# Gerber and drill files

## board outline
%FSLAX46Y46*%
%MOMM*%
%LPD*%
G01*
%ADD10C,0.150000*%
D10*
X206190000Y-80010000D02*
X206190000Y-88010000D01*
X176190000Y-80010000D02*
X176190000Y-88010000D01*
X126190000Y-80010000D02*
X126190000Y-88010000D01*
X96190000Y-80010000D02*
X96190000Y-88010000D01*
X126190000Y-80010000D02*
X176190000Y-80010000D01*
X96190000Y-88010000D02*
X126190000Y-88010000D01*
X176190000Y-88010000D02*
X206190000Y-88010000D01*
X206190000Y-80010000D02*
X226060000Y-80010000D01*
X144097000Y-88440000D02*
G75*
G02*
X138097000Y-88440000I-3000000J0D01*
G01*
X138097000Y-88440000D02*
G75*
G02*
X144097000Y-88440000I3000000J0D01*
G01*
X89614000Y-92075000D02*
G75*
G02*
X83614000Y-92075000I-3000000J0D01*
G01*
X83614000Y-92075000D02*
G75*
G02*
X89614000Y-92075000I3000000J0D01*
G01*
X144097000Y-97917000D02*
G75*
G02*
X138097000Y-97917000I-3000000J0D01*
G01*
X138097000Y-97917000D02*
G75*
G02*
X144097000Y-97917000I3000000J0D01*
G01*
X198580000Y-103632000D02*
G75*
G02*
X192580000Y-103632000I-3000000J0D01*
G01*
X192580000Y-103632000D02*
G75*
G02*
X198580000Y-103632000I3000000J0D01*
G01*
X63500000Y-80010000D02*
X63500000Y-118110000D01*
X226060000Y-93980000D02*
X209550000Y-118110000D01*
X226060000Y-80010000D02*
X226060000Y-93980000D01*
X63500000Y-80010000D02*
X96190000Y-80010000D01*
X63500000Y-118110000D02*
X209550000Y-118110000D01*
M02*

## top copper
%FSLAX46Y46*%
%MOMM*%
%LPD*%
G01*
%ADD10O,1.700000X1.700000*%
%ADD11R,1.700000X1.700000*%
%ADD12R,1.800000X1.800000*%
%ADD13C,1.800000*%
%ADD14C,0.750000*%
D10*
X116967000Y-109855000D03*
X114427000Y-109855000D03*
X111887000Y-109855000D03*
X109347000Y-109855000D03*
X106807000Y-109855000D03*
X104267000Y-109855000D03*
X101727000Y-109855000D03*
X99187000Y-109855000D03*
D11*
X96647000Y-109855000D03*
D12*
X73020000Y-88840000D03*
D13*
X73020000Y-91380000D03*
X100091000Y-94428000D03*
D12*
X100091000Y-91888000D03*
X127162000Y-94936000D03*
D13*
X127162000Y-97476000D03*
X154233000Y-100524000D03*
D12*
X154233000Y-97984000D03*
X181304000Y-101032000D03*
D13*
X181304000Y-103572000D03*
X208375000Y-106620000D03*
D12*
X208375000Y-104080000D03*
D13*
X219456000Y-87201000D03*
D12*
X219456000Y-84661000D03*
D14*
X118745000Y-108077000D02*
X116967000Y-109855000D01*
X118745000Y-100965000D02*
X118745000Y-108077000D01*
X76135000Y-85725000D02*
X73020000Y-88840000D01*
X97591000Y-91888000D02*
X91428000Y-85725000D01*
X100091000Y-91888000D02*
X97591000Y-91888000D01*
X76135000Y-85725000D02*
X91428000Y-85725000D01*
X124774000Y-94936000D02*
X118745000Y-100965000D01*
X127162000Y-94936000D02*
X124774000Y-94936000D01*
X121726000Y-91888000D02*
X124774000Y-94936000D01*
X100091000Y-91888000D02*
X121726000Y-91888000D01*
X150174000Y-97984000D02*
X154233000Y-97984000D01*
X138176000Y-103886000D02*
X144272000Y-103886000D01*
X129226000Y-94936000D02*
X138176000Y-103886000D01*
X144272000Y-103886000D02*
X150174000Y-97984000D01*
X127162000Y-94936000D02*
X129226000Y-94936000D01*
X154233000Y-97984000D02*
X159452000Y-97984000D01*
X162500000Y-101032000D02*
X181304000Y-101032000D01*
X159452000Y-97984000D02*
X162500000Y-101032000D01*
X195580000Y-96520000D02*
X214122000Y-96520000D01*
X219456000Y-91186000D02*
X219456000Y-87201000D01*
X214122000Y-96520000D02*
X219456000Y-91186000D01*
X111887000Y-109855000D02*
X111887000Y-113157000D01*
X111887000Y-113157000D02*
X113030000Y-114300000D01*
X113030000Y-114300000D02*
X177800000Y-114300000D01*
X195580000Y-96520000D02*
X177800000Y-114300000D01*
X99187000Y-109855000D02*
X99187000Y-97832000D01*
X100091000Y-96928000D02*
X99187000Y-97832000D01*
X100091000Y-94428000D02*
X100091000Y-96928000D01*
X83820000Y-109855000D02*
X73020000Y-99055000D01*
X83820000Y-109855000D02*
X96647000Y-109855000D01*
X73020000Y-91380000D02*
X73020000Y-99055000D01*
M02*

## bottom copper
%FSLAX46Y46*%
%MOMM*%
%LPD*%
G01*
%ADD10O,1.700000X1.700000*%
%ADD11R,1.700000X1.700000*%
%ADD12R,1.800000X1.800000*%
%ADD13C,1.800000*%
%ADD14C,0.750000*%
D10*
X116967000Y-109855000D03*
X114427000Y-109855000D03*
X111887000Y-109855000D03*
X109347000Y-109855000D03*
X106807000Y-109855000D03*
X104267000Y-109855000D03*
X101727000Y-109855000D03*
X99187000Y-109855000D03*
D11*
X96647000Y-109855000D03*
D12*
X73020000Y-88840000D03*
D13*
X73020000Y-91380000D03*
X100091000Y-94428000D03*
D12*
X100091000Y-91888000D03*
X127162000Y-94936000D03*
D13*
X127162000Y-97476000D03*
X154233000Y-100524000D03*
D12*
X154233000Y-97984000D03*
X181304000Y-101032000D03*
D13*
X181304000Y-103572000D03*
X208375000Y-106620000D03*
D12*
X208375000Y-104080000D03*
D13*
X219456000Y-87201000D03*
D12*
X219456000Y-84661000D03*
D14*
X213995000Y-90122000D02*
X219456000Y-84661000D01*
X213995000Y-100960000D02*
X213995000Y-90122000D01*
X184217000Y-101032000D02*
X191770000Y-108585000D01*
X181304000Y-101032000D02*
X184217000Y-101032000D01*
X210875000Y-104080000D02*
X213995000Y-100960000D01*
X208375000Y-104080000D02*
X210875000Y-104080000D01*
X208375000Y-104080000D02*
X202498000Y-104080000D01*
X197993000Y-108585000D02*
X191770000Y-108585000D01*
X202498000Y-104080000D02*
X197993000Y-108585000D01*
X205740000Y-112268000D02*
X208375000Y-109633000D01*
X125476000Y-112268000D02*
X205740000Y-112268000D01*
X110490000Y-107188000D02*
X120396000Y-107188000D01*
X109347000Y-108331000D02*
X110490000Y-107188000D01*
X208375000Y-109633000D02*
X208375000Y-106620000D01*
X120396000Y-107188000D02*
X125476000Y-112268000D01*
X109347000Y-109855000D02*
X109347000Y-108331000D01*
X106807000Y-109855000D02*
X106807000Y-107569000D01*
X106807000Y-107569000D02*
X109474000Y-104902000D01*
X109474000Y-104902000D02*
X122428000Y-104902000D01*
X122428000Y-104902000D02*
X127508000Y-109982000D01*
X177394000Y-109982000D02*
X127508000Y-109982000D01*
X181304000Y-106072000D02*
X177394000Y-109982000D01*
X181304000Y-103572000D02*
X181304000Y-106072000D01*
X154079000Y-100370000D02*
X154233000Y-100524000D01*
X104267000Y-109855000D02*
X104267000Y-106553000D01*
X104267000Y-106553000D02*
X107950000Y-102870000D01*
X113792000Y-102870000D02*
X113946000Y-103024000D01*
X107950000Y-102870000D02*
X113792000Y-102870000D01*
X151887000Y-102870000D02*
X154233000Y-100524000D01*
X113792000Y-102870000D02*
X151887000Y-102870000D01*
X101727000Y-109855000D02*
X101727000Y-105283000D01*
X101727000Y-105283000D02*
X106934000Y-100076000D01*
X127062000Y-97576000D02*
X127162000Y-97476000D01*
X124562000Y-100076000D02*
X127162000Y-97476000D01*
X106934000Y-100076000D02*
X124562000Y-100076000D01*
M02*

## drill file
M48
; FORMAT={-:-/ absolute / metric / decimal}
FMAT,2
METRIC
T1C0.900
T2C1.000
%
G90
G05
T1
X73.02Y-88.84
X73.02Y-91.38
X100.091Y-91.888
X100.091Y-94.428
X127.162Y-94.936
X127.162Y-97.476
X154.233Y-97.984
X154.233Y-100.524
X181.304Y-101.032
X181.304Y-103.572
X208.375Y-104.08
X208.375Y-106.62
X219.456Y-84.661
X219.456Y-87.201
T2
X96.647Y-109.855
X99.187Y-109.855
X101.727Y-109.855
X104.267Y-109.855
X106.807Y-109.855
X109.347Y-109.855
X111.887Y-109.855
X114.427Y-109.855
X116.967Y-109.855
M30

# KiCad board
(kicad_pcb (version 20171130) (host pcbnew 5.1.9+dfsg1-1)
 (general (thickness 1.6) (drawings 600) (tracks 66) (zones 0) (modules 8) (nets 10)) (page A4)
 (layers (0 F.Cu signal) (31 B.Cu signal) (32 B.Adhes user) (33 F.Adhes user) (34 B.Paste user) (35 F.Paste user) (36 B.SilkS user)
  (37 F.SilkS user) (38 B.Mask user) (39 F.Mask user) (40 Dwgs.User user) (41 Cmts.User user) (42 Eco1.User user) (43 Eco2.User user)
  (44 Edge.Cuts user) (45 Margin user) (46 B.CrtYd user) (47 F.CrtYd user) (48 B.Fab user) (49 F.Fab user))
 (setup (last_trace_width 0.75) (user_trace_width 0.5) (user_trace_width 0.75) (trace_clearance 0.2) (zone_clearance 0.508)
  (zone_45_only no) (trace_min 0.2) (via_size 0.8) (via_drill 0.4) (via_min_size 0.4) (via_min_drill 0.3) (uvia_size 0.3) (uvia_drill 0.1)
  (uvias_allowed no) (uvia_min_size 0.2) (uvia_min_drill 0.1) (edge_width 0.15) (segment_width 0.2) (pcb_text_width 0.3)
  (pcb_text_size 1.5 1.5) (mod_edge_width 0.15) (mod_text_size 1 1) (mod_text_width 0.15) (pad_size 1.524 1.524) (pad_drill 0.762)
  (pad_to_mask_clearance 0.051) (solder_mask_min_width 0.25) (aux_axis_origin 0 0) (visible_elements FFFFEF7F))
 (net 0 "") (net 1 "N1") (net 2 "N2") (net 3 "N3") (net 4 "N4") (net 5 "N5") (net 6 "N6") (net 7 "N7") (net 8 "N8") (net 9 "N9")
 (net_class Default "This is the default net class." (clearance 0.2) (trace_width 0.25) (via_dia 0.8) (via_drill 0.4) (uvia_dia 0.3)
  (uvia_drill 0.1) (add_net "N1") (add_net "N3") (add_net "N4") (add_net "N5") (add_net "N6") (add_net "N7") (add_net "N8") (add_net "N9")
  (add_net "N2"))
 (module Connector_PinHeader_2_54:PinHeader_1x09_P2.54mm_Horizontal (layer B.Cu) (at 96.647 109.855 270)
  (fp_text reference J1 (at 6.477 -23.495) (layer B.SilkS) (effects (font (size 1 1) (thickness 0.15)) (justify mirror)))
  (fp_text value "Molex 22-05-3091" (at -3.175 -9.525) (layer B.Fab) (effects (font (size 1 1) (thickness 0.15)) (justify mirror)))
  (pad 9 thru_hole oval (at 0 -20.32 270) (size 1.7 1.7) (drill 1) (layers *.Cu *.Mask) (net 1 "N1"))
  (pad 8 thru_hole oval (at 0 -17.78 270) (size 1.7 1.7) (drill 1) (layers *.Cu *.Mask) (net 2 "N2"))
  (pad 7 thru_hole oval (at 0 -15.24 270) (size 1.7 1.7) (drill 1) (layers *.Cu *.Mask) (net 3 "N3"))
  (pad 6 thru_hole oval (at 0 -12.7 270) (size 1.7 1.7) (drill 1) (layers *.Cu *.Mask) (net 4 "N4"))
  (pad 5 thru_hole oval (at 0 -10.16 270) (size 1.7 1.7) (drill 1) (layers *.Cu *.Mask) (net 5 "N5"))
  (pad 4 thru_hole oval (at 0 -7.62 270) (size 1.7 1.7) (drill 1) (layers *.Cu *.Mask) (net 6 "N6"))
  (pad 3 thru_hole oval (at 0 -5.08 270) (size 1.7 1.7) (drill 1) (layers *.Cu *.Mask) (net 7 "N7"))
  (pad 2 thru_hole oval (at 0 -2.54 270) (size 1.7 1.7) (drill 1) (layers *.Cu *.Mask) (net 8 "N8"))
  (pad 1 thru_hole rect (at 0 0 270) (size 1.7 1.7) (drill 1) (layers *.Cu *.Mask) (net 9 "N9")))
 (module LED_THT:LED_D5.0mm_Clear (layer B.Cu) (at 73.02 88.84 270)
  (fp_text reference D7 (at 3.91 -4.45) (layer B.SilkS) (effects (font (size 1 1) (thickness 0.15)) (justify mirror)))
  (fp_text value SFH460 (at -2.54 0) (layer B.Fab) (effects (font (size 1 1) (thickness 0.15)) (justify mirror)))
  (pad 1 thru_hole rect (at 0 0 270) (size 1.8 1.8) (drill 0.9) (layers *.Cu *.Mask) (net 1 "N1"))
  (pad 2 thru_hole circle (at 2.54 0 270) (size 1.8 1.8) (drill 0.9) (layers *.Cu *.Mask) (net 9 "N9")))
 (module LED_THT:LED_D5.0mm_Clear (layer B.Cu) (at 100.091 91.888 270)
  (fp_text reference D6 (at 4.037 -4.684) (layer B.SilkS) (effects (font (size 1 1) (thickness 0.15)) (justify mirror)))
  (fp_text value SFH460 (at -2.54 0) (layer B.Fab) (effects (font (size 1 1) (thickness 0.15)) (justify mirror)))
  (pad 2 thru_hole circle (at 2.54 0 270) (size 1.8 1.8) (drill 0.9) (layers *.Cu *.Mask) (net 8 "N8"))
  (pad 1 thru_hole rect (at 0 0 270) (size 1.8 1.8) (drill 0.9) (layers *.Cu *.Mask) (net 1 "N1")))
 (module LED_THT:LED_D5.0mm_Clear (layer B.Cu) (at 127.162 94.936 270)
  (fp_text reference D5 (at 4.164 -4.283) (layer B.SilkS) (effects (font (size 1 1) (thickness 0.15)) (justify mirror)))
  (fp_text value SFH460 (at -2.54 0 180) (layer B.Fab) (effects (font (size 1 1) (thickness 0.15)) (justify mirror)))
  (pad 1 thru_hole rect (at 0 0 270) (size 1.8 1.8) (drill 0.9) (layers *.Cu *.Mask) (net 1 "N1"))
  (pad 2 thru_hole circle (at 2.54 0 270) (size 1.8 1.8) (drill 0.9) (layers *.Cu *.Mask) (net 7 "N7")))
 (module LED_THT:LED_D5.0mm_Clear (layer B.Cu) (at 154.233 97.984 270)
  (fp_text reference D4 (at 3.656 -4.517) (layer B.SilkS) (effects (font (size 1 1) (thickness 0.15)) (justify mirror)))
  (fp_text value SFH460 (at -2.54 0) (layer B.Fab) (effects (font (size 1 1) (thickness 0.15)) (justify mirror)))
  (pad 2 thru_hole circle (at 2.54 0 270) (size 1.8 1.8) (drill 0.9) (layers *.Cu *.Mask) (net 6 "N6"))
  (pad 1 thru_hole rect (at 0 0 270) (size 1.8 1.8) (drill 0.9) (layers *.Cu *.Mask) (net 1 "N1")))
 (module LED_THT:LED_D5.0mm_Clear (layer B.Cu) (at 181.304 101.032 270)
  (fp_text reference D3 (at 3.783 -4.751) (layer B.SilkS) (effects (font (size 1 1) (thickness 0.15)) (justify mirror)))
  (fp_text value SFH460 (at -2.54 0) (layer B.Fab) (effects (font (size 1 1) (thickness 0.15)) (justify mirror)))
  (pad 1 thru_hole rect (at 0 0 270) (size 1.8 1.8) (drill 0.9) (layers *.Cu *.Mask) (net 1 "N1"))
  (pad 2 thru_hole circle (at 2.54 0 270) (size 1.8 1.8) (drill 0.9) (layers *.Cu *.Mask) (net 5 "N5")))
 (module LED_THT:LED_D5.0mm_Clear (layer B.Cu) (at 208.375 104.08 270)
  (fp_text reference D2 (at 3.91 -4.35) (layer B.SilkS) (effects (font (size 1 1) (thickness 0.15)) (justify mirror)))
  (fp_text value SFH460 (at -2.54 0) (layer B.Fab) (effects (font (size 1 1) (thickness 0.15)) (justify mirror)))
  (pad 2 thru_hole circle (at 2.54 0 270) (size 1.8 1.8) (drill 0.9) (layers *.Cu *.Mask) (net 4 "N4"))
  (pad 1 thru_hole rect (at 0 0 270) (size 1.8 1.8) (drill 0.9) (layers *.Cu *.Mask) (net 1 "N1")))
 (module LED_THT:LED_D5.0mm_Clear (layer B.Cu) (at 219.456 84.661 270)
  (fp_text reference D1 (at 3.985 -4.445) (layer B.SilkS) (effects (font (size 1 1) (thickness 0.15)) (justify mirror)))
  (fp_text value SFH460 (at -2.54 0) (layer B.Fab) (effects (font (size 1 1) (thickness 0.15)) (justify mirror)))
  (pad 2 thru_hole circle (at 2.54 0 270) (size 1.8 1.8) (drill 0.9) (layers *.Cu *.Mask) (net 3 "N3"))
  (pad 1 thru_hole rect (at 0 0 270) (size 1.8 1.8) (drill 0.9) (layers *.Cu *.Mask) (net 1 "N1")))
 (gr_line (start 206.19 80.01) (end 206.19 88.01) (layer Edge.Cuts) (width 0.15))
 (gr_line (start 176.19 80.01) (end 176.19 88.01) (layer Edge.Cuts) (width 0.15))
 (gr_line (start 126.19 80.01) (end 126.19 88.01) (layer Edge.Cuts) (width 0.15))
 (gr_line (start 96.19 80.01) (end 96.19 88.01) (layer Edge.Cuts) (width 0.15))
 (gr_line (start 126.19 80.01) (end 176.19 80.01) (layer Edge.Cuts) (width 0.15))
 (gr_line (start 96.19 88.01) (end 126.19 88.01) (layer Edge.Cuts) (width 0.15))
 (gr_line (start 176.19 88.01) (end 206.19 88.01) (layer Edge.Cuts) (width 0.15))
 (gr_line (start 206.19 80.01) (end 226.06 80.01) (layer Edge.Cuts) (width 0.15))
 (gr_circle (center 141.097 88.44) (end 144.097 88.44) (layer Edge.Cuts) (width 0.15))
 (gr_circle (center 86.614 92.075) (end 89.614 92.075) (layer Edge.Cuts) (width 0.15))
 (gr_circle (center 141.097 97.917) (end 144.097 97.917) (layer Edge.Cuts) (width 0.15))
 (gr_circle (center 195.58 103.632) (end 198.58 103.632) (layer Edge.Cuts) (width 0.15))
 (gr_line (start 63.5 80.01) (end 63.5 118.11) (layer Edge.Cuts) (width 0.15))
 (gr_line (start 226.06 93.98) (end 209.55 118.11) (layer Edge.Cuts) (width 0.15))
 (gr_line (start 226.06 80.01) (end 226.06 93.98) (layer Edge.Cuts) (width 0.15))
 (gr_line (start 63.5 80.01) (end 96.19 80.01) (layer Edge.Cuts) (width 0.15))
 (gr_line (start 63.5 118.11) (end 209.55 118.11) (layer Edge.Cuts) (width 0.15))
 (segment (start 213.995 90.122) (end 219.456 84.661) (width 0.75) (layer B.Cu) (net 1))
 (segment (start 213.995 100.96) (end 213.995 90.122) (width 0.75) (layer B.Cu) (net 1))
 (segment (start 118.745 108.077) (end 116.967 109.855) (width 0.75) (layer F.Cu) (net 1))
 (segment (start 118.745 100.965) (end 118.745 108.077) (width 0.75) (layer F.Cu) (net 1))
 (segment (start 76.135 85.725) (end 73.02 88.84) (width 0.75) (layer F.Cu) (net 1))
 (segment (start 97.591 91.888) (end 91.428 85.725) (width 0.75) (layer F.Cu) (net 1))
 (segment (start 100.091 91.888) (end 97.591 91.888) (width 0.75) (layer F.Cu) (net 1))
 (segment (start 76.135 85.725) (end 91.428 85.725) (width 0.75) (layer F.Cu) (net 1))
 (segment (start 124.774 94.936) (end 118.745 100.965) (width 0.75) (layer F.Cu) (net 1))
 (segment (start 127.162 94.936) (end 124.774 94.936) (width 0.75) (layer F.Cu) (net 1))
 (segment (start 121.726 91.888) (end 124.774 94.936) (width 0.75) (layer F.Cu) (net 1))
 (segment (start 100.091 91.888) (end 121.726 91.888) (width 0.75) (layer F.Cu) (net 1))
 (segment (start 150.174 97.984) (end 154.233 97.984) (width 0.75) (layer F.Cu) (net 1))
 (segment (start 138.176 103.886) (end 144.272 103.886) (width 0.75) (layer F.Cu) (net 1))
 (segment (start 129.226 94.936) (end 138.176 103.886) (width 0.75) (layer F.Cu) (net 1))
 (segment (start 144.272 103.886) (end 150.174 97.984) (width 0.75) (layer F.Cu) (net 1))
 (segment (start 127.162 94.936) (end 129.226 94.936) (width 0.75) (layer F.Cu) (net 1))
 (segment (start 154.233 97.984) (end 159.452 97.984) (width 0.75) (layer F.Cu) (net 1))
 (segment (start 162.5 101.032) (end 181.304 101.032) (width 0.75) (layer F.Cu) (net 1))
 (segment (start 159.452 97.984) (end 162.5 101.032) (width 0.75) (layer F.Cu) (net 1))
 (segment (start 184.217 101.032) (end 191.77 108.585) (width 0.75) (layer B.Cu) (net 1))
 (segment (start 181.304 101.032) (end 184.217 101.032) (width 0.75) (layer B.Cu) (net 1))
 (segment (start 210.875 104.08) (end 213.995 100.96) (width 0.75) (layer B.Cu) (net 1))
 (segment (start 208.375 104.08) (end 210.875 104.08) (width 0.75) (layer B.Cu) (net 1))
 (segment (start 208.375 104.08) (end 202.498 104.08) (width 0.75) (layer B.Cu) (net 1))
 (segment (start 197.993 108.585) (end 191.77 108.585) (width 0.75) (layer B.Cu) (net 1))
 (segment (start 202.498 104.08) (end 197.993 108.585) (width 0.75) (layer B.Cu) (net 1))
 (segment (start 195.58 96.52) (end 214.122 96.52) (width 0.75) (layer F.Cu) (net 3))
 (segment (start 219.456 91.186) (end 219.456 87.201) (width 0.75) (layer F.Cu) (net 3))
 (segment (start 214.122 96.52) (end 219.456 91.186) (width 0.75) (layer F.Cu) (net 3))
 (segment (start 111.887 109.855) (end 111.887 113.157) (width 0.75) (layer F.Cu) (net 3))
 (segment (start 111.887 113.157) (end 113.03 114.3) (width 0.75) (layer F.Cu) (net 3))
 (segment (start 113.03 114.3) (end 177.8 114.3) (width 0.75) (layer F.Cu) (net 3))
 (segment (start 195.58 96.52) (end 177.8 114.3) (width 0.75) (layer F.Cu) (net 3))
 (segment (start 205.74 112.268) (end 208.375 109.633) (width 0.75) (layer B.Cu) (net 4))
 (segment (start 125.476 112.268) (end 205.74 112.268) (width 0.75) (layer B.Cu) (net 4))
 (segment (start 110.49 107.188) (end 120.396 107.188) (width 0.75) (layer B.Cu) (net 4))
 (segment (start 109.347 108.331) (end 110.49 107.188) (width 0.75) (layer B.Cu) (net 4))
 (segment (start 208.375 109.633) (end 208.375 106.62) (width 0.75) (layer B.Cu) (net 4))
 (segment (start 120.396 107.188) (end 125.476 112.268) (width 0.75) (layer B.Cu) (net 4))
 (segment (start 109.347 109.855) (end 109.347 108.331) (width 0.75) (layer B.Cu) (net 4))
 (segment (start 106.807 109.855) (end 106.807 107.569) (width 0.75) (layer B.Cu) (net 5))
 (segment (start 106.807 107.569) (end 109.474 104.902) (width 0.75) (layer B.Cu) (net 5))
 (segment (start 109.474 104.902) (end 122.428 104.902) (width 0.75) (layer B.Cu) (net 5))
 (segment (start 122.428 104.902) (end 127.508 109.982) (width 0.75) (layer B.Cu) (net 5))
 (segment (start 177.394 109.982) (end 127.508 109.982) (width 0.75) (layer B.Cu) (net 5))
 (segment (start 181.304 106.072) (end 177.394 109.982) (width 0.75) (layer B.Cu) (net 5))
 (segment (start 181.304 103.572) (end 181.304 106.072) (width 0.75) (layer B.Cu) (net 5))
 (segment (start 154.079 100.37) (end 154.233 100.524) (width 0.75) (layer B.Cu) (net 6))
 (segment (start 104.267 109.855) (end 104.267 106.553) (width 0.75) (layer B.Cu) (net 6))
 (segment (start 104.267 106.553) (end 107.95 102.87) (width 0.75) (layer B.Cu) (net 6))
 (segment (start 113.792 102.87) (end 113.946 103.024) (width 0.75) (layer B.Cu) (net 6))
 (segment (start 107.95 102.87) (end 113.792 102.87) (width 0.75) (layer B.Cu) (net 6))
 (segment (start 151.887 102.87) (end 154.233 100.524) (width 0.75) (layer B.Cu) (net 6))
 (segment (start 113.792 102.87) (end 151.887 102.87) (width 0.75) (layer B.Cu) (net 6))
 (segment (start 101.727 109.855) (end 101.727 105.283) (width 0.75) (layer B.Cu) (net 7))
 (segment (start 101.727 105.283) (end 106.934 100.076) (width 0.75) (layer B.Cu) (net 7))
 (segment (start 127.062 97.576) (end 127.162 97.476) (width 0.75) (layer B.Cu) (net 7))
 (segment (start 124.562 100.076) (end 127.162 97.476) (width 0.75) (layer B.Cu) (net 7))
 (segment (start 106.934 100.076) (end 124.562 100.076) (width 0.75) (layer B.Cu) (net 7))
 (segment (start 99.187 109.855) (end 99.187 97.832) (width 0.75) (layer F.Cu) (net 8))
 (segment (start 100.091 96.928) (end 99.187 97.832) (width 0.75) (layer F.Cu) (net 8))
 (segment (start 100.091 94.428) (end 100.091 96.928) (width 0.75) (layer F.Cu) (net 8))
 (segment (start 83.82 109.855) (end 73.02 99.055) (width 0.75) (layer F.Cu) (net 9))
 (segment (start 83.82 109.855) (end 96.647 109.855) (width 0.75) (layer F.Cu) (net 9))
 (segment (start 73.02 91.38) (end 73.02 99.055) (width 0.75) (layer F.Cu) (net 9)))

